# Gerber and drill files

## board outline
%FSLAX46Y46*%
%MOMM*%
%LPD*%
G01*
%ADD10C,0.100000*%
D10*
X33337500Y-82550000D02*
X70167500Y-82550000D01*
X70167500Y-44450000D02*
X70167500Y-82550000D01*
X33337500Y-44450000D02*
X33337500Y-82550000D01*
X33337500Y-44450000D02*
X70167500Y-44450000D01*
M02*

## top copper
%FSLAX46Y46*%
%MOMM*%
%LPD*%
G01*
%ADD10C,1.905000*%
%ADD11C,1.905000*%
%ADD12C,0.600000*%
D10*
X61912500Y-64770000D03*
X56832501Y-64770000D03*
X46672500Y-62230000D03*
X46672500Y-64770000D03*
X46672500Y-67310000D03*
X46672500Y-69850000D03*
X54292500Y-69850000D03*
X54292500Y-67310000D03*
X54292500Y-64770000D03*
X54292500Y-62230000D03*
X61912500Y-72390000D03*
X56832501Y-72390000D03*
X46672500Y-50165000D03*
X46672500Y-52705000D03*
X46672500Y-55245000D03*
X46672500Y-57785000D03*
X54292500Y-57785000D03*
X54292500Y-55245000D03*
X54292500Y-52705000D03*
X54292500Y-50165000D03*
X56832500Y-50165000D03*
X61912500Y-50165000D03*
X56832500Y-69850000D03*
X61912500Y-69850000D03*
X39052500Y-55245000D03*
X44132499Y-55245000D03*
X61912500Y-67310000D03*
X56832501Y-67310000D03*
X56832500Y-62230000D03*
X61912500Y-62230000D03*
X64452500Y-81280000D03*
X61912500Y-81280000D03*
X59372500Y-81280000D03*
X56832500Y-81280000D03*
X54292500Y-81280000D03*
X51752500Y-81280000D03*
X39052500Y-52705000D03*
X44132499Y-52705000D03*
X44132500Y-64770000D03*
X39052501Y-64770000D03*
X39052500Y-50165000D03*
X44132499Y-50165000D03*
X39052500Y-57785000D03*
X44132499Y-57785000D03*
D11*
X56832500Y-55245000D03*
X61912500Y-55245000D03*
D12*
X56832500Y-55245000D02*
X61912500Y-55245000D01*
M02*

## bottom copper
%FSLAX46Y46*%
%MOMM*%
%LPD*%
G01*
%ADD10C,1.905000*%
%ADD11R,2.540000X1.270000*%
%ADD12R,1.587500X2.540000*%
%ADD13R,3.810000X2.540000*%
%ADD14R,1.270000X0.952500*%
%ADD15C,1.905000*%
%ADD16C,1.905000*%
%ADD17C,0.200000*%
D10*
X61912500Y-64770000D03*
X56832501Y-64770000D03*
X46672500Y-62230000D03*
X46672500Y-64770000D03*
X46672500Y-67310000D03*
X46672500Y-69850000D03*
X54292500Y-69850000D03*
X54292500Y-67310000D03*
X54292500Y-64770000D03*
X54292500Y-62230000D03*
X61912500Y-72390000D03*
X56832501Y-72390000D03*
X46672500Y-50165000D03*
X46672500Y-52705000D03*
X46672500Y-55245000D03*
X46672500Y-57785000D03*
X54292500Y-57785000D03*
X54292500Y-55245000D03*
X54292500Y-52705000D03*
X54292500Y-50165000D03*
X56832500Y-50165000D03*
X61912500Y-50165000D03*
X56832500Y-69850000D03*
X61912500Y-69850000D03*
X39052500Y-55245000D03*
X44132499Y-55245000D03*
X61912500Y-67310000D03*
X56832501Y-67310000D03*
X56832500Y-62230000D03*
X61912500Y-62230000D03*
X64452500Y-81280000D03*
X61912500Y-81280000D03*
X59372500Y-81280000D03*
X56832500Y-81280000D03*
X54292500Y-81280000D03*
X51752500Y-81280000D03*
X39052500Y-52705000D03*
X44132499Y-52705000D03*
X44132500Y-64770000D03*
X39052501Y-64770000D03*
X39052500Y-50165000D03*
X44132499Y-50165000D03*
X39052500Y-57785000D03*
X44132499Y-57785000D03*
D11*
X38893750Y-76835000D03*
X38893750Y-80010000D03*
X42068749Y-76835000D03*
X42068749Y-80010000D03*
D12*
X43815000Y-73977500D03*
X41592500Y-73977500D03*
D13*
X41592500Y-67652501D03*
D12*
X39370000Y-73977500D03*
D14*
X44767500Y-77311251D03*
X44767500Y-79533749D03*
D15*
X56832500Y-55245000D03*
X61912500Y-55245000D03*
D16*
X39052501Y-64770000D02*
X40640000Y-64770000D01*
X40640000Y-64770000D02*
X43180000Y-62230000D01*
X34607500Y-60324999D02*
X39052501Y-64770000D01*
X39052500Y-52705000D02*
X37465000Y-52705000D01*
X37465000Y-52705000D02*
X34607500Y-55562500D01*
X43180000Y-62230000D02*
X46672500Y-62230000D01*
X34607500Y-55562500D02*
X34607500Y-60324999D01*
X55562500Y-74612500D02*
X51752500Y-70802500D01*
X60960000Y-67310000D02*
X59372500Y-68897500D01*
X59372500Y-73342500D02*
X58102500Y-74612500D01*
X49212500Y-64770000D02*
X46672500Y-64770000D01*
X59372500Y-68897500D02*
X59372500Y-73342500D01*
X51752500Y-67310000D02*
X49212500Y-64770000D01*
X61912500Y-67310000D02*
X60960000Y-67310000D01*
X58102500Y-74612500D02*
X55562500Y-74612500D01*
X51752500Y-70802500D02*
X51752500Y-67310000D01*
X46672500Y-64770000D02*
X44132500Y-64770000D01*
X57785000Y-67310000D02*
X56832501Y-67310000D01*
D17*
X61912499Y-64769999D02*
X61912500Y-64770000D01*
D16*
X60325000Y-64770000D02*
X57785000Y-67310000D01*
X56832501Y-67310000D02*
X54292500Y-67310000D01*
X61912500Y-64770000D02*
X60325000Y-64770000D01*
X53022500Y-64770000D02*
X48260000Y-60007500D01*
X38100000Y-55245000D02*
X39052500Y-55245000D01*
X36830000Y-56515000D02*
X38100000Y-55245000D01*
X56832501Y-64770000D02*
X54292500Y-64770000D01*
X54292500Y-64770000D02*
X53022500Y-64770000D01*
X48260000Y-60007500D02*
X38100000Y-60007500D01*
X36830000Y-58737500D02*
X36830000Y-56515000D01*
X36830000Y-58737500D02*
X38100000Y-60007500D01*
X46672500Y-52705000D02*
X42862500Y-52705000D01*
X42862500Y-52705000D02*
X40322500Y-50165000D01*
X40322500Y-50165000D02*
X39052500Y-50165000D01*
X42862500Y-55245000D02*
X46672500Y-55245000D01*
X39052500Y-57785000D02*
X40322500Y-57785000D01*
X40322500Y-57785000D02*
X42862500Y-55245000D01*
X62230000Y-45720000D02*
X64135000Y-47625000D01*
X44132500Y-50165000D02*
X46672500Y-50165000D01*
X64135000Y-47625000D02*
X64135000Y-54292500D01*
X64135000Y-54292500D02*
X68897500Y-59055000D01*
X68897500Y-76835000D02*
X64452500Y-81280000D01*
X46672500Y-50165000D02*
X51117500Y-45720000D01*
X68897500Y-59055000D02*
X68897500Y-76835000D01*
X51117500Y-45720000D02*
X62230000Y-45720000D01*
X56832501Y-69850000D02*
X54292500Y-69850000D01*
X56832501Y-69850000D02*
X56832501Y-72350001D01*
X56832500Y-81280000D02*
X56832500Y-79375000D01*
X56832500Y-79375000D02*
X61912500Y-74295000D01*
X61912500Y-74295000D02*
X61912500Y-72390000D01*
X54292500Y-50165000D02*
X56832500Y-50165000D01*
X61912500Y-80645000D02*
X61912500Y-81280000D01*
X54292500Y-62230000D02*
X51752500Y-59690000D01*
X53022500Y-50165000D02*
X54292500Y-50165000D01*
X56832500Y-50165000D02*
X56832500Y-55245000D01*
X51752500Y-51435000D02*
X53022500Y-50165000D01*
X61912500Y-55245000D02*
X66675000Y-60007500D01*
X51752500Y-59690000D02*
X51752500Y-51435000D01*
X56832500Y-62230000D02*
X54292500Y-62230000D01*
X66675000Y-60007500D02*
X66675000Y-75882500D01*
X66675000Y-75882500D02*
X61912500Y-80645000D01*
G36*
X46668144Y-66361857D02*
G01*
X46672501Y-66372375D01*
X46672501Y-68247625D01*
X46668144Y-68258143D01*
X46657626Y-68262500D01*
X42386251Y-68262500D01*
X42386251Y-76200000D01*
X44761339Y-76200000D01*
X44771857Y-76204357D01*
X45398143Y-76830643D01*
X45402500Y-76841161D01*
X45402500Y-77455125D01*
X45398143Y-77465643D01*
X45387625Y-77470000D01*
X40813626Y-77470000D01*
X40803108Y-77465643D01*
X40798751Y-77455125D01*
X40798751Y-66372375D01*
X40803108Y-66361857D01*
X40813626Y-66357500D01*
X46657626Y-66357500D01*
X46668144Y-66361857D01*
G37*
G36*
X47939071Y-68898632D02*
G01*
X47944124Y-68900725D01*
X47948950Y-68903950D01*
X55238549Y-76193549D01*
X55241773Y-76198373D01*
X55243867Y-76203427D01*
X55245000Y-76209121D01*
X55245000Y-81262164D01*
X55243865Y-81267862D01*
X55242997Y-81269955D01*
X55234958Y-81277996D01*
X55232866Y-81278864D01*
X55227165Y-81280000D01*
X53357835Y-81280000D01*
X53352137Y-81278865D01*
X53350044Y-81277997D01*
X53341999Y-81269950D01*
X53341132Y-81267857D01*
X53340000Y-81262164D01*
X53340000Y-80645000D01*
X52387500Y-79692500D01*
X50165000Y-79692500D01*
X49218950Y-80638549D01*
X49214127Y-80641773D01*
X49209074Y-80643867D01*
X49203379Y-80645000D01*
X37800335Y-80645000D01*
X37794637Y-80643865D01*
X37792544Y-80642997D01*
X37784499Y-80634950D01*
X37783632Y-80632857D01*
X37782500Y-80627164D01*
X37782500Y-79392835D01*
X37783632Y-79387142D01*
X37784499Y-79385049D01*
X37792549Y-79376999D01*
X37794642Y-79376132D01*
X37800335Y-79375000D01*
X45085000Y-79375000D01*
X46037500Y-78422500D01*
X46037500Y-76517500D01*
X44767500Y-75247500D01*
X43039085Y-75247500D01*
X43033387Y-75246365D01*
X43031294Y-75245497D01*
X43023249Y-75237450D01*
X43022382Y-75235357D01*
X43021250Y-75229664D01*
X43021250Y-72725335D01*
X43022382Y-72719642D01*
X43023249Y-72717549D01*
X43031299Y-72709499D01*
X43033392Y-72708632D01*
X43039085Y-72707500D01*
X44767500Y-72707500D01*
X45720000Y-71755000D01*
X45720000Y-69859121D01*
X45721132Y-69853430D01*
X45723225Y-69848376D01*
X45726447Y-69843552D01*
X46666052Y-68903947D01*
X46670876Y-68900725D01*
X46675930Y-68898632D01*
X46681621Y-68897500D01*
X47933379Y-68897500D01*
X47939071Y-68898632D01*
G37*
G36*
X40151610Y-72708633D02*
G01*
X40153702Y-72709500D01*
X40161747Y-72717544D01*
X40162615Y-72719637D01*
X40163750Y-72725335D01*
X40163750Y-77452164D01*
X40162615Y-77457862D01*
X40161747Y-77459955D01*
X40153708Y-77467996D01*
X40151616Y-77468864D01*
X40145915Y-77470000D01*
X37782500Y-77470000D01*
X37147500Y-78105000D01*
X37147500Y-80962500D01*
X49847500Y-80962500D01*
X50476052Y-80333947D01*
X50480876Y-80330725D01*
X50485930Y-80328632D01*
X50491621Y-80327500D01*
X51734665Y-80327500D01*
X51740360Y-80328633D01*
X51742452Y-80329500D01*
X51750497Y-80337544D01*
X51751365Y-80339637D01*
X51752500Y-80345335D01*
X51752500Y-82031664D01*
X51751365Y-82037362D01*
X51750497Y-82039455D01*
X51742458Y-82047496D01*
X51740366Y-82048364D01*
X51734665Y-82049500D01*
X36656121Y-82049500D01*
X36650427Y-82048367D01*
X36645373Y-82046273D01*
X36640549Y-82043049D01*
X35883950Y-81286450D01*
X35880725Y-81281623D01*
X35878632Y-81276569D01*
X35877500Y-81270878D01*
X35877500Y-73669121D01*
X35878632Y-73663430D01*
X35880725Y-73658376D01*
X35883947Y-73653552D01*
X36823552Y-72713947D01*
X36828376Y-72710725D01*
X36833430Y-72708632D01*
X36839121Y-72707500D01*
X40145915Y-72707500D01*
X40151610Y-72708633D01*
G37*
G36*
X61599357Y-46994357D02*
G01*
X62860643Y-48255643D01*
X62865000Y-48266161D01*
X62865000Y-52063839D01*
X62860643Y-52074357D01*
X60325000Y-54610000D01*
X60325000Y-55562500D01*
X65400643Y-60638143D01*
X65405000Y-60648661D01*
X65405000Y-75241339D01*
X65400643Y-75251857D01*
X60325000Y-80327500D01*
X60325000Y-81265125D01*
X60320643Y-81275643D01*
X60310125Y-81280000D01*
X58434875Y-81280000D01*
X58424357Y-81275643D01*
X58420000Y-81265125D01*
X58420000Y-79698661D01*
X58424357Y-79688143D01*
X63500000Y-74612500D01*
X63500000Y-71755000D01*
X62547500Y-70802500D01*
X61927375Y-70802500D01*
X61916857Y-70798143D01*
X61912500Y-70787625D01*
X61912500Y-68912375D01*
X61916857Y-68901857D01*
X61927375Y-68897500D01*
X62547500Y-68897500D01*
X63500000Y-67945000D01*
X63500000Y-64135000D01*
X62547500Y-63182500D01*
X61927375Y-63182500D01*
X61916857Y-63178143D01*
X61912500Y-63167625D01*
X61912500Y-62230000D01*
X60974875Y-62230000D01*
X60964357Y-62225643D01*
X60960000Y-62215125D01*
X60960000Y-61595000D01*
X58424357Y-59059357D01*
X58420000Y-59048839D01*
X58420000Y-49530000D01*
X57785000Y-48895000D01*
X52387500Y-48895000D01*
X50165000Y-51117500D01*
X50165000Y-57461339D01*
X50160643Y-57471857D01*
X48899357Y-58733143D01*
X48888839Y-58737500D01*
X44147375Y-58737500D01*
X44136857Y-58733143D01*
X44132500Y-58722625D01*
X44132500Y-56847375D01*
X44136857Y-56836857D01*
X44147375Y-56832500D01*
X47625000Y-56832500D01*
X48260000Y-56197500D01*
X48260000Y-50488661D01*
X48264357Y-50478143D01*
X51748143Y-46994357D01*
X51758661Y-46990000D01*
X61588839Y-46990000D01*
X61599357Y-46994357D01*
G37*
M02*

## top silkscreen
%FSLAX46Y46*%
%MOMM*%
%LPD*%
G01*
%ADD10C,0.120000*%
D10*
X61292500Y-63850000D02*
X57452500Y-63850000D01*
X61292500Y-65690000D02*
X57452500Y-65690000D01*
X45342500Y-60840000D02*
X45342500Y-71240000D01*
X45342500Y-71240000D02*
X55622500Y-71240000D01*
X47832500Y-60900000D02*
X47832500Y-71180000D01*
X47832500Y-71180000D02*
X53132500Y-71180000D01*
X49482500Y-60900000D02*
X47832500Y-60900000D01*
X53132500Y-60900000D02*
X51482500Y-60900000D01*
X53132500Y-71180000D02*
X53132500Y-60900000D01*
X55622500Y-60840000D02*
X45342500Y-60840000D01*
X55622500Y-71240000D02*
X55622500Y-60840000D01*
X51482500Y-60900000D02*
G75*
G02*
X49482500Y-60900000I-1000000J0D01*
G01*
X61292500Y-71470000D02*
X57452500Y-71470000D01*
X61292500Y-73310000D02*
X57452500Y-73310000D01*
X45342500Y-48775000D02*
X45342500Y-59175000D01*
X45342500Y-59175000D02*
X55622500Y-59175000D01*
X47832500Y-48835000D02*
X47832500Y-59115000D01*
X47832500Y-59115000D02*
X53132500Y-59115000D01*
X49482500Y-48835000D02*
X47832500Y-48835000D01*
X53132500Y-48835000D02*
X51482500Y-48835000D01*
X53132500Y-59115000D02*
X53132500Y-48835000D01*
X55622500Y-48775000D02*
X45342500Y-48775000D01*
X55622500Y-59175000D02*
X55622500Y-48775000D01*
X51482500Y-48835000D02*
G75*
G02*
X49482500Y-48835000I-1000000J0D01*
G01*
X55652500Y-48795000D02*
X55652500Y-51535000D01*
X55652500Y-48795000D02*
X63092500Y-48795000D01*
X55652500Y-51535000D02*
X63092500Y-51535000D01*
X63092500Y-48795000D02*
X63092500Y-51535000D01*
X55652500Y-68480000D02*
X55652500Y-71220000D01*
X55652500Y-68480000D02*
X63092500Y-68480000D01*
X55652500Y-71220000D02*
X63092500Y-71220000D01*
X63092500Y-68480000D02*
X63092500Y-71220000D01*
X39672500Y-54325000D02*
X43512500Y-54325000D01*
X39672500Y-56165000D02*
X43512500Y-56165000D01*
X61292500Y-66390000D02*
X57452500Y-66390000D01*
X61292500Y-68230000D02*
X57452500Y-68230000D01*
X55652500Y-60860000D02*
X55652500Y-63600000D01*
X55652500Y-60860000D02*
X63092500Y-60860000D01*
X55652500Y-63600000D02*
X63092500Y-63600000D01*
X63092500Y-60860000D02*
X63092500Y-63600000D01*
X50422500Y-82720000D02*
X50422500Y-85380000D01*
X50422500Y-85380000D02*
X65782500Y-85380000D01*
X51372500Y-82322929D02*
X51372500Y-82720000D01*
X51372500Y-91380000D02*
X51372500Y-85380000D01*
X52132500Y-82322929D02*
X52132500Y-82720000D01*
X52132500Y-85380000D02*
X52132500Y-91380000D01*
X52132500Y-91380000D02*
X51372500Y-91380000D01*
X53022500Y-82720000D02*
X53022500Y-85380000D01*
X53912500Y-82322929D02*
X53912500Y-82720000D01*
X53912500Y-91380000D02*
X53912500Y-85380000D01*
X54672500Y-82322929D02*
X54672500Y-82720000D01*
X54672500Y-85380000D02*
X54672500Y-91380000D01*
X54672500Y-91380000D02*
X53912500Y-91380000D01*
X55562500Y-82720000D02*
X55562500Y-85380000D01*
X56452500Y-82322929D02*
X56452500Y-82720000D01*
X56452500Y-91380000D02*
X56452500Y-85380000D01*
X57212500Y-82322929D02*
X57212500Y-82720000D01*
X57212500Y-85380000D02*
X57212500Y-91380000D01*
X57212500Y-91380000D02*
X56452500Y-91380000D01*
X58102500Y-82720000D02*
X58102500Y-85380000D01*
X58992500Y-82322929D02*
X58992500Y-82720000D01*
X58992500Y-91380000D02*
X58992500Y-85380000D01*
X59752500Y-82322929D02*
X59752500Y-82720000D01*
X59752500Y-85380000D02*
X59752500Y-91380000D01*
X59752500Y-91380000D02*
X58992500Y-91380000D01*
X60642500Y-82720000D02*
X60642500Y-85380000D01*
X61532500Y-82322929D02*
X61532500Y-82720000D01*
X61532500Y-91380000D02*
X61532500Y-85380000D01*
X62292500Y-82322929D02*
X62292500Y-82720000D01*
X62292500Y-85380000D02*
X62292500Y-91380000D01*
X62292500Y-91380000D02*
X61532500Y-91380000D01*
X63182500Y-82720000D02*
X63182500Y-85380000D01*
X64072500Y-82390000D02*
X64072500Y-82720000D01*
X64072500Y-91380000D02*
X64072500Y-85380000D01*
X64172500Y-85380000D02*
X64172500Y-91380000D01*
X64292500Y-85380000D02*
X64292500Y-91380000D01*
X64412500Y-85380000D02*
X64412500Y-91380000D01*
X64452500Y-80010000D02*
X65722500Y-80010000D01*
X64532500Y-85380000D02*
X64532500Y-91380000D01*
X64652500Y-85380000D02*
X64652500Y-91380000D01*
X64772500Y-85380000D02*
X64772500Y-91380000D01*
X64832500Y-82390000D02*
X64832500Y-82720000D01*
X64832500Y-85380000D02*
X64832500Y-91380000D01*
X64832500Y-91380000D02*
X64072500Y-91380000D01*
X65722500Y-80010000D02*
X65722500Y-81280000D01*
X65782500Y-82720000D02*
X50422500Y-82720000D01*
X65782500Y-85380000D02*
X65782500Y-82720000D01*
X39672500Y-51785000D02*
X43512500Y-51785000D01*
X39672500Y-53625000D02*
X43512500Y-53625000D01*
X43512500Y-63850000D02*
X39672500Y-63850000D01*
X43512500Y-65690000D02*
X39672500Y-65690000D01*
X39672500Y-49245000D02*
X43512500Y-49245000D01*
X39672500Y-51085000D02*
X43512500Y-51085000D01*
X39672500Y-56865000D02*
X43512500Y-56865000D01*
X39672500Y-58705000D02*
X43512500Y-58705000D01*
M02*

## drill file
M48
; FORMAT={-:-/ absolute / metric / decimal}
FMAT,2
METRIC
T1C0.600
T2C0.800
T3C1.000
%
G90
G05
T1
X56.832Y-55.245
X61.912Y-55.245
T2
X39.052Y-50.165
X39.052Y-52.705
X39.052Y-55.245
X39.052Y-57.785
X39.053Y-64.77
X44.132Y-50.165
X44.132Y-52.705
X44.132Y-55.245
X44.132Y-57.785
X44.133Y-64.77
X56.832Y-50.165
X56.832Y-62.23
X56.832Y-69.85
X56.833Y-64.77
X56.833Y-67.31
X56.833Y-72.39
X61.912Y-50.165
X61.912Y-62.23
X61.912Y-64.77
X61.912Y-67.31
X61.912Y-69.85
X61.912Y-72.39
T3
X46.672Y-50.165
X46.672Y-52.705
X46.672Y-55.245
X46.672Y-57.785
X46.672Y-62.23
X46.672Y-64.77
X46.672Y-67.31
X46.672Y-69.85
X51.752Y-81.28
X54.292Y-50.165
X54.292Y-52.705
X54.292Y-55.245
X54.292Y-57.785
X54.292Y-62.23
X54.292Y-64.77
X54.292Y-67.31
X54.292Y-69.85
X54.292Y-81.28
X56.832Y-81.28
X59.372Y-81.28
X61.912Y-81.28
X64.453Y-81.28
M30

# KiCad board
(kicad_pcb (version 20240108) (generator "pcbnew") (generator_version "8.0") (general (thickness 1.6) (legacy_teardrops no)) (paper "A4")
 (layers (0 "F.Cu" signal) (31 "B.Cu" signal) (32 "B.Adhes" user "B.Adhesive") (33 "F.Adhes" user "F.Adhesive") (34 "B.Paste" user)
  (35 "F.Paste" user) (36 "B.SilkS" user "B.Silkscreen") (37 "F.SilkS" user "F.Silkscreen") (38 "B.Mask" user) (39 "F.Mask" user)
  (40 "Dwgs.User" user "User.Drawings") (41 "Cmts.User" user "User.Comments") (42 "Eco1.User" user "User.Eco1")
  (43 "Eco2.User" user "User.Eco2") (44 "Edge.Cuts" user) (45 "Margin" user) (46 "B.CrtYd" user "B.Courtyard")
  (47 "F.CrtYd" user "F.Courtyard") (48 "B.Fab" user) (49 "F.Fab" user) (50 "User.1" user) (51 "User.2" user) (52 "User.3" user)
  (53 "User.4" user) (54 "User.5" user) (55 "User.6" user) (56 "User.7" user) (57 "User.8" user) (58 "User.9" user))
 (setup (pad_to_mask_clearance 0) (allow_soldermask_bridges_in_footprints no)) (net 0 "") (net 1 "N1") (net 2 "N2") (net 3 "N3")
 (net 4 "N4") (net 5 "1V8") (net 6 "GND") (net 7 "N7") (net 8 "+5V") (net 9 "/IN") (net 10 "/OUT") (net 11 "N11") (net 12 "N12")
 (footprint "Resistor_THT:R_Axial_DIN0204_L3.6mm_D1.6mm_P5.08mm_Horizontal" (layer "F.Cu") (at 61.9125 64.77 180)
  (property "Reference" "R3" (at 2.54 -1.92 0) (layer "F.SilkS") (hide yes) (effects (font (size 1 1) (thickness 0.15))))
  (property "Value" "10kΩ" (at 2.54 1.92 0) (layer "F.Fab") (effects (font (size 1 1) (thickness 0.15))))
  (fp_line (start 0.62 0.92) (end 4.46 0.92) (stroke (width 0.12) (type solid)) (layer "F.SilkS"))
  (fp_line (start 0.62 -0.92) (end 4.46 -0.92) (stroke (width 0.12) (type solid)) (layer "F.SilkS"))
  (pad "1" thru_hole circle (at 0 0 180) (size 1.905 1.905) (drill 0.8) (layers "*.Cu" "*.Mask") (remove_unused_layers no) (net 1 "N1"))
  (pad "2" thru_hole circle (at 5.079999 0 180) (size 1.905 1.905) (drill 0.8) (layers "*.Cu" "*.Mask") (remove_unused_layers no)
   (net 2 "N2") (thermal_bridge_angle 90)))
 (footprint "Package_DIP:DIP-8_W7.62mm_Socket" (layer "F.Cu") (at 50.4825 66.04)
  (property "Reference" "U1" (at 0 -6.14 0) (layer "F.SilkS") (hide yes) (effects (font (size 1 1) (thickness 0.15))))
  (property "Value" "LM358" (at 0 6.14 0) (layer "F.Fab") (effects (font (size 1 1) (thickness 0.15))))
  (fp_line (start -5.14 -5.2) (end -5.14 5.2) (stroke (width 0.12) (type solid)) (layer "F.SilkS"))
  (fp_line (start -5.14 5.2) (end 5.14 5.2) (stroke (width 0.12) (type solid)) (layer "F.SilkS"))
  (fp_line (start -2.65 -5.14) (end -2.65 5.14) (stroke (width 0.12) (type solid)) (layer "F.SilkS"))
  (fp_line (start -2.65 5.14) (end 2.65 5.14) (stroke (width 0.12) (type solid)) (layer "F.SilkS"))
  (fp_line (start -1 -5.14) (end -2.65 -5.14) (stroke (width 0.12) (type solid)) (layer "F.SilkS"))
  (fp_line (start 2.65 -5.14) (end 1 -5.14) (stroke (width 0.12) (type solid)) (layer "F.SilkS"))
  (fp_line (start 2.65 5.14) (end 2.65 -5.14) (stroke (width 0.12) (type solid)) (layer "F.SilkS"))
  (fp_line (start 5.14 -5.2) (end -5.14 -5.2) (stroke (width 0.12) (type solid)) (layer "F.SilkS"))
  (fp_line (start 5.14 5.2) (end 5.14 -5.2) (stroke (width 0.12) (type solid)) (layer "F.SilkS"))
  (fp_arc (start 1 -5.14) (mid 0 -4.14) (end -1 -5.14) (stroke (width 0.12) (type solid)) (layer "F.SilkS"))
  (pad "1" thru_hole circle (at -3.81 -3.81) (size 1.905 1.905) (drill 1) (layers "*.Cu" "*.Mask") (remove_unused_layers no) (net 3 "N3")
   (thermal_bridge_angle 90))
  (pad "2" thru_hole circle (at -3.81 -1.27) (size 1.905 1.905) (drill 1) (layers "*.Cu" "*.Mask") (remove_unused_layers no) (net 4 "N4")
   (thermal_bridge_angle 90))
  (pad "3" thru_hole circle (at -3.81 1.27) (size 1.905 1.905) (drill 1) (layers "*.Cu" "*.Mask") (remove_unused_layers no) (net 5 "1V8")
   (thermal_bridge_angle 90))
  (pad "4" thru_hole circle (at -3.81 3.81) (size 1.905 1.905) (drill 1) (layers "*.Cu" "*.Mask") (remove_unused_layers no) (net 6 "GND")
   (thermal_bridge_angle 90))
  (pad "5" thru_hole circle (at 3.81 3.81) (size 1.905 1.905) (drill 1) (layers "*.Cu" "*.Mask") (remove_unused_layers no) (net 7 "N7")
   (thermal_bridge_angle 90))
  (pad "6" thru_hole circle (at 3.81 1.27) (size 1.905 1.905) (drill 1) (layers "*.Cu" "*.Mask") (remove_unused_layers no) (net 1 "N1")
   (thermal_bridge_angle 90))
  (pad "7" thru_hole circle (at 3.81 -1.27) (size 1.905 1.905) (drill 1) (layers "*.Cu" "*.Mask") (remove_unused_layers no) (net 2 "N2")
   (thermal_bridge_angle 90))
  (pad "8" thru_hole circle (at 3.81 -3.81) (size 1.905 1.905) (drill 1) (layers "*.Cu" "*.Mask") (remove_unused_layers no) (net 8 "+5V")
   (thermal_bridge_angle 90)))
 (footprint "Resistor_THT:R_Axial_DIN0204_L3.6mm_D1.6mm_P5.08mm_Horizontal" (layer "F.Cu") (at 61.9125 72.39 180)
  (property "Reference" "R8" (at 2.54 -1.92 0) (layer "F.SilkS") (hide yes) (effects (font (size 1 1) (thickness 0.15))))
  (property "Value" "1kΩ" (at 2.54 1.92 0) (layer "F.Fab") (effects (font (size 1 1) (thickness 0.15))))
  (fp_line (start 0.62 0.92) (end 4.46 0.92) (stroke (width 0.12) (type solid)) (layer "F.SilkS"))
  (fp_line (start 0.62 -0.92) (end 4.46 -0.92) (stroke (width 0.12) (type solid)) (layer "F.SilkS"))
  (pad "1" thru_hole circle (at 0 0 180) (size 1.905 1.905) (drill 0.8) (layers "*.Cu" "*.Mask") (remove_unused_layers no) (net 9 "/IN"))
  (pad "2" thru_hole circle (at 5.079999 0 180) (size 1.905 1.905) (drill 0.8) (layers "*.Cu" "*.Mask") (remove_unused_layers no)
   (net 7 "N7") (thermal_bridge_angle 90)))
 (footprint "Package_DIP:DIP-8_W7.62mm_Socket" (layer "F.Cu") (at 50.4825 53.975)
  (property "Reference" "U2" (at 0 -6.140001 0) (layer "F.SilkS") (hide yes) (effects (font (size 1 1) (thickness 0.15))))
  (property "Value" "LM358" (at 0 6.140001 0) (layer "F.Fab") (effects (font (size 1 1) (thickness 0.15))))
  (fp_line (start -5.14 -5.2) (end -5.14 5.2) (stroke (width 0.12) (type solid)) (layer "F.SilkS"))
  (fp_line (start -5.14 5.2) (end 5.14 5.2) (stroke (width 0.12) (type solid)) (layer "F.SilkS"))
  (fp_line (start -2.65 -5.14) (end -2.65 5.14) (stroke (width 0.12) (type solid)) (layer "F.SilkS"))
  (fp_line (start -2.65 5.14) (end 2.65 5.14) (stroke (width 0.12) (type solid)) (layer "F.SilkS"))
  (fp_line (start -1 -5.14) (end -2.65 -5.14) (stroke (width 0.12) (type solid)) (layer "F.SilkS"))
  (fp_line (start 2.65 -5.14) (end 1 -5.14) (stroke (width 0.12) (type solid)) (layer "F.SilkS"))
  (fp_line (start 2.65 5.14) (end 2.65 -5.14) (stroke (width 0.12) (type solid)) (layer "F.SilkS"))
  (fp_line (start 5.14 -5.2) (end -5.14 -5.2) (stroke (width 0.12) (type solid)) (layer "F.SilkS"))
  (fp_line (start 5.14 5.2) (end 5.14 -5.2) (stroke (width 0.12) (type solid)) (layer "F.SilkS"))
  (fp_arc (start 1 -5.14) (mid 0 -4.14) (end -1 -5.14) (stroke (width 0.12) (type solid)) (layer "F.SilkS"))
  (pad "1" thru_hole circle (at -3.81 -3.81) (size 1.905 1.905) (drill 1) (layers "*.Cu" "*.Mask") (remove_unused_layers no) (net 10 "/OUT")
   (thermal_bridge_angle 90))
  (pad "2" thru_hole circle (at -3.81 -1.27) (size 1.905 1.905) (drill 1) (layers "*.Cu" "*.Mask") (remove_unused_layers no) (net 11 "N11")
   (thermal_bridge_angle 90))
  (pad "3" thru_hole circle (at -3.81 1.27) (size 1.905 1.905) (drill 1) (layers "*.Cu" "*.Mask") (remove_unused_layers no) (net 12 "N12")
   (thermal_bridge_angle 90))
  (pad "4" thru_hole circle (at -3.81 3.81) (size 1.905 1.905) (drill 1) (layers "*.Cu" "*.Mask") (remove_unused_layers no) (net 6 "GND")
   (thermal_bridge_angle 90))
  (pad "5" thru_hole circle (at 3.81 3.81) (size 1.905 1.905) (drill 1) (layers "*.Cu" "*.Mask") (remove_unused_layers no)
   (thermal_bridge_angle 90))
  (pad "6" thru_hole circle (at 3.81 1.27) (size 1.905 1.905) (drill 1) (layers "*.Cu" "*.Mask") (remove_unused_layers no)
   (thermal_bridge_angle 90))
  (pad "7" thru_hole circle (at 3.81 -1.27) (size 1.905 1.905) (drill 1) (layers "*.Cu" "*.Mask") (remove_unused_layers no)
   (thermal_bridge_angle 90))
  (pad "8" thru_hole circle (at 3.81 -3.81) (size 1.905 1.905) (drill 1) (layers "*.Cu" "*.Mask") (remove_unused_layers no) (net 8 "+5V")
   (thermal_bridge_angle 90)))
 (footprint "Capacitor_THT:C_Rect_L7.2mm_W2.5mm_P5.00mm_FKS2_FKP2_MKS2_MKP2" (layer "F.Cu") (at 56.8725 50.165)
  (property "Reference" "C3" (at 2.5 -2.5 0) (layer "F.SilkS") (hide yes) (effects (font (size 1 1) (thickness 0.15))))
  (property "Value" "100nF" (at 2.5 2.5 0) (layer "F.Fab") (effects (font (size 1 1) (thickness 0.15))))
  (fp_line (start -1.22 -1.37) (end -1.22 1.37) (stroke (width 0.12) (type solid)) (layer "F.SilkS"))
  (fp_line (start -1.22 -1.37) (end 6.22 -1.37) (stroke (width 0.12) (type solid)) (layer "F.SilkS"))
  (fp_line (start -1.22 1.37) (end 6.22 1.37) (stroke (width 0.12) (type solid)) (layer "F.SilkS"))
  (fp_line (start 6.22 -1.37) (end 6.22 1.37) (stroke (width 0.12) (type solid)) (layer "F.SilkS"))
  (pad "1" thru_hole circle (at -0.04 0) (size 1.905 1.6) (drill 0.8) (layers "*.Cu" "*.Mask") (remove_unused_layers no) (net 8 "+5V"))
  (pad "2" thru_hole circle (at 5.04 0) (size 1.905 1.6) (drill 0.8) (layers "*.Cu" "*.Mask") (remove_unused_layers no) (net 6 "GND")))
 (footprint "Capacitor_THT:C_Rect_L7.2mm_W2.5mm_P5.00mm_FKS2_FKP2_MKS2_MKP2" (layer "F.Cu") (at 56.8725 69.85)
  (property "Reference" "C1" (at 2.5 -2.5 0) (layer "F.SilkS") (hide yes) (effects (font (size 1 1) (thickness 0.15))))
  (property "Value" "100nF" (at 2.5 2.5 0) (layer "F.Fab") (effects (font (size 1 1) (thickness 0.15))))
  (fp_line (start -1.22 -1.37) (end -1.22 1.37) (stroke (width 0.12) (type solid)) (layer "F.SilkS"))
  (fp_line (start -1.22 -1.37) (end 6.22 -1.37) (stroke (width 0.12) (type solid)) (layer "F.SilkS"))
  (fp_line (start -1.22 1.37) (end 6.22 1.37) (stroke (width 0.12) (type solid)) (layer "F.SilkS"))
  (fp_line (start 6.22 -1.37) (end 6.22 1.37) (stroke (width 0.12) (type solid)) (layer "F.SilkS"))
  (pad "1" thru_hole circle (at -0.04 0) (size 1.905 1.6) (drill 0.8) (layers "*.Cu" "*.Mask") (remove_unused_layers no) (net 7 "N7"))
  (pad "2" thru_hole circle (at 5.04 0) (size 1.905 1.6) (drill 0.8) (layers "*.Cu" "*.Mask") (remove_unused_layers no) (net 6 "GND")))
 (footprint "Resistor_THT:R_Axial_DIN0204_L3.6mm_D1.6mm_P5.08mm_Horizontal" (layer "F.Cu") (at 39.0525 55.245)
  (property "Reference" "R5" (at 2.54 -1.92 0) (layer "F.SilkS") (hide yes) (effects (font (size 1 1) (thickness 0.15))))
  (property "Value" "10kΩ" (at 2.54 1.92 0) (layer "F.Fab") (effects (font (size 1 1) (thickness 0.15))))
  (fp_line (start 0.62 -0.92) (end 4.46 -0.92) (stroke (width 0.12) (type solid)) (layer "F.SilkS"))
  (fp_line (start 0.62 0.92) (end 4.46 0.92) (stroke (width 0.12) (type solid)) (layer "F.SilkS"))
  (pad "1" thru_hole circle (at 0 0) (size 1.905 1.905) (drill 0.8) (layers "*.Cu" "*.Mask") (remove_unused_layers no) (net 2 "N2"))
  (pad "2" thru_hole circle (at 5.079999 0) (size 1.905 1.905) (drill 0.8) (layers "*.Cu" "*.Mask") (remove_unused_layers no) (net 12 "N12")
   (thermal_bridge_angle 90)))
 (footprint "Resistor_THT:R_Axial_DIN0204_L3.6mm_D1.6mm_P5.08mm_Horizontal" (layer "F.Cu") (at 61.9125 67.31 180)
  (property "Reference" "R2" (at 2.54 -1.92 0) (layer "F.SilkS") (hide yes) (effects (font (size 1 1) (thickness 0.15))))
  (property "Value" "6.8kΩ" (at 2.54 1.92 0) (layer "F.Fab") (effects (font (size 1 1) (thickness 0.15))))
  (fp_line (start 0.62 0.92) (end 4.46 0.92) (stroke (width 0.12) (type solid)) (layer "F.SilkS"))
  (fp_line (start 0.62 -0.92) (end 4.46 -0.92) (stroke (width 0.12) (type solid)) (layer "F.SilkS"))
  (pad "1" thru_hole circle (at 0 0 180) (size 1.905 1.905) (drill 0.8) (layers "*.Cu" "*.Mask") (remove_unused_layers no) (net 4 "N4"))
  (pad "2" thru_hole circle (at 5.079999 0 180) (size 1.905 1.905) (drill 0.8) (layers "*.Cu" "*.Mask") (remove_unused_layers no)
   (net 1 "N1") (thermal_bridge_angle 90)))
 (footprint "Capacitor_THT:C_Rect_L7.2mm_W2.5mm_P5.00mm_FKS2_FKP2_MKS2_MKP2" (layer "F.Cu") (at 56.8725 62.23)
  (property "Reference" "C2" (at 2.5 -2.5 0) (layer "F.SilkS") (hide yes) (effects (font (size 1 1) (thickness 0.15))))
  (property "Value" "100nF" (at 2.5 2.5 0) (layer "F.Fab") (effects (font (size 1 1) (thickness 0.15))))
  (fp_line (start -1.22 -1.37) (end -1.22 1.37) (stroke (width 0.12) (type solid)) (layer "F.SilkS"))
  (fp_line (start -1.22 -1.37) (end 6.22 -1.37) (stroke (width 0.12) (type solid)) (layer "F.SilkS"))
  (fp_line (start -1.22 1.37) (end 6.22 1.37) (stroke (width 0.12) (type solid)) (layer "F.SilkS"))
  (fp_line (start 6.22 -1.37) (end 6.22 1.37) (stroke (width 0.12) (type solid)) (layer "F.SilkS"))
  (pad "1" thru_hole circle (at -0.04 0) (size 1.905 1.6) (drill 0.8) (layers "*.Cu" "*.Mask") (remove_unused_layers no) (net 8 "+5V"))
  (pad "2" thru_hole circle (at 5.04 0) (size 1.905 1.6) (drill 0.8) (layers "*.Cu" "*.Mask") (remove_unused_layers no) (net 6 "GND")))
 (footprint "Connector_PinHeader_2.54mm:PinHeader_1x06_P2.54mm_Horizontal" (layer "F.Cu") (at 64.4525 81.28 -90)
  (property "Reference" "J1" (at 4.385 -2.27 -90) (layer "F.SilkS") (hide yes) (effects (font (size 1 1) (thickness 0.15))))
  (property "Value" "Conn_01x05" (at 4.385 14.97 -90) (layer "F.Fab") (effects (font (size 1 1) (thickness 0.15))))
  (fp_line (start 1.44 14.03) (end 4.1 14.03) (stroke (width 0.12) (type solid)) (layer "F.SilkS"))
  (fp_line (start 4.1 14.03) (end 4.1 -1.33) (stroke (width 0.12) (type solid)) (layer "F.SilkS"))
  (fp_line (start 1.042929 13.08) (end 1.44 13.08) (stroke (width 0.12) (type solid)) (layer "F.SilkS"))
  (fp_line (start 10.1 13.08) (end 4.1 13.08) (stroke (width 0.12) (type solid)) (layer "F.SilkS"))
  (fp_line (start 1.042929 12.32) (end 1.44 12.32) (stroke (width 0.12) (type solid)) (layer "F.SilkS"))
  (fp_line (start 4.1 12.32) (end 10.1 12.32) (stroke (width 0.12) (type solid)) (layer "F.SilkS"))
  (fp_line (start 10.1 12.32) (end 10.1 13.08) (stroke (width 0.12) (type solid)) (layer "F.SilkS"))
  (fp_line (start 1.44 11.43) (end 4.1 11.43) (stroke (width 0.12) (type solid)) (layer "F.SilkS"))
  (fp_line (start 1.042929 10.54) (end 1.44 10.54) (stroke (width 0.12) (type solid)) (layer "F.SilkS"))
  (fp_line (start 10.1 10.54) (end 4.1 10.54) (stroke (width 0.12) (type solid)) (layer "F.SilkS"))
  (fp_line (start 1.042929 9.78) (end 1.44 9.78) (stroke (width 0.12) (type solid)) (layer "F.SilkS"))
  (fp_line (start 4.1 9.78) (end 10.1 9.78) (stroke (width 0.12) (type solid)) (layer "F.SilkS"))
  (fp_line (start 10.1 9.78) (end 10.1 10.54) (stroke (width 0.12) (type solid)) (layer "F.SilkS"))
  (fp_line (start 1.44 8.89) (end 4.1 8.89) (stroke (width 0.12) (type solid)) (layer "F.SilkS"))
  (fp_line (start 1.042929 8) (end 1.44 8) (stroke (width 0.12) (type solid)) (layer "F.SilkS"))
  (fp_line (start 10.1 8) (end 4.1 8) (stroke (width 0.12) (type solid)) (layer "F.SilkS"))
  (fp_line (start 1.042929 7.24) (end 1.44 7.24) (stroke (width 0.12) (type solid)) (layer "F.SilkS"))
  (fp_line (start 4.1 7.24) (end 10.1 7.24) (stroke (width 0.12) (type solid)) (layer "F.SilkS"))
  (fp_line (start 10.1 7.24) (end 10.1 8) (stroke (width 0.12) (type solid)) (layer "F.SilkS"))
  (fp_line (start 1.44 6.35) (end 4.1 6.35) (stroke (width 0.12) (type solid)) (layer "F.SilkS"))
  (fp_line (start 1.042929 5.46) (end 1.44 5.46) (stroke (width 0.12) (type solid)) (layer "F.SilkS"))
  (fp_line (start 10.1 5.46) (end 4.1 5.46) (stroke (width 0.12) (type solid)) (layer "F.SilkS"))
  (fp_line (start 1.042929 4.7) (end 1.44 4.7) (stroke (width 0.12) (type solid)) (layer "F.SilkS"))
  (fp_line (start 4.1 4.7) (end 10.1 4.7) (stroke (width 0.12) (type solid)) (layer "F.SilkS"))
  (fp_line (start 10.1 4.7) (end 10.1 5.46) (stroke (width 0.12) (type solid)) (layer "F.SilkS"))
  (fp_line (start 1.44 3.81) (end 4.1 3.81) (stroke (width 0.12) (type solid)) (layer "F.SilkS"))
  (fp_line (start 1.042929 2.92) (end 1.44 2.92) (stroke (width 0.12) (type solid)) (layer "F.SilkS"))
  (fp_line (start 10.1 2.92) (end 4.1 2.92) (stroke (width 0.12) (type solid)) (layer "F.SilkS"))
  (fp_line (start 1.042929 2.16) (end 1.44 2.16) (stroke (width 0.12) (type solid)) (layer "F.SilkS"))
  (fp_line (start 4.1 2.16) (end 10.1 2.16) (stroke (width 0.12) (type solid)) (layer "F.SilkS"))
  (fp_line (start 10.1 2.16) (end 10.1 2.92) (stroke (width 0.12) (type solid)) (layer "F.SilkS"))
  (fp_line (start 1.44 1.27) (end 4.1 1.27) (stroke (width 0.12) (type solid)) (layer "F.SilkS"))
  (fp_line (start 1.11 0.38) (end 1.44 0.38) (stroke (width 0.12) (type solid)) (layer "F.SilkS"))
  (fp_line (start 10.1 0.38) (end 4.1 0.38) (stroke (width 0.12) (type solid)) (layer "F.SilkS"))
  (fp_line (start 4.1 0.28) (end 10.1 0.28) (stroke (width 0.12) (type solid)) (layer "F.SilkS"))
  (fp_line (start 4.1 0.16) (end 10.1 0.16) (stroke (width 0.12) (type solid)) (layer "F.SilkS"))
  (fp_line (start 4.1 0.04) (end 10.1 0.04) (stroke (width 0.12) (type solid)) (layer "F.SilkS"))
  (fp_line (start -1.27 0) (end -1.27 -1.27) (stroke (width 0.12) (type solid)) (layer "F.SilkS"))
  (fp_line (start 4.1 -0.08) (end 10.1 -0.08) (stroke (width 0.12) (type solid)) (layer "F.SilkS"))
  (fp_line (start 4.1 -0.2) (end 10.1 -0.2) (stroke (width 0.12) (type solid)) (layer "F.SilkS"))
  (fp_line (start 4.1 -0.32) (end 10.1 -0.32) (stroke (width 0.12) (type solid)) (layer "F.SilkS"))
  (fp_line (start 1.11 -0.38) (end 1.44 -0.38) (stroke (width 0.12) (type solid)) (layer "F.SilkS"))
  (fp_line (start 4.1 -0.38) (end 10.1 -0.38) (stroke (width 0.12) (type solid)) (layer "F.SilkS"))
  (fp_line (start 10.1 -0.38) (end 10.1 0.38) (stroke (width 0.12) (type solid)) (layer "F.SilkS"))
  (fp_line (start -1.27 -1.27) (end 0 -1.27) (stroke (width 0.12) (type solid)) (layer "F.SilkS"))
  (fp_line (start 1.44 -1.33) (end 1.44 14.03) (stroke (width 0.12) (type solid)) (layer "F.SilkS"))
  (fp_line (start 4.1 -1.33) (end 1.44 -1.33) (stroke (width 0.12) (type solid)) (layer "F.SilkS"))
  (pad "1" thru_hole circle (at 0 0 270) (size 1.905 1.905) (drill 1) (layers "*.Cu" "*.Mask") (remove_unused_layers no) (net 10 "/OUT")
   (thermal_bridge_angle 90))
  (pad "2" thru_hole circle (at 0 2.54 270) (size 1.905 1.905) (drill 1) (layers "*.Cu" "*.Mask") (remove_unused_layers no) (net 8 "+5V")
   (thermal_bridge_angle 90))
  (pad "3" thru_hole circle (at 0 5.08 270) (size 1.905 1.905) (drill 1) (layers "*.Cu" "*.Mask") (remove_unused_layers no) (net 6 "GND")
   (thermal_bridge_angle 90))
  (pad "4" thru_hole circle (at 0 7.62 270) (size 1.905 1.905) (drill 1) (layers "*.Cu" "*.Mask") (remove_unused_layers no) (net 9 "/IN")
   (thermal_bridge_angle 90))
  (pad "5" thru_hole circle (at 0 10.16 270) (size 1.905 1.905) (drill 1) (layers "*.Cu" "*.Mask") (remove_unused_layers no) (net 6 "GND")
   (thermal_bridge_angle 90))
  (pad "6" thru_hole circle (at 0 12.7 270) (size 1.905 1.905) (drill 1) (layers "*.Cu" "*.Mask") (remove_unused_layers no) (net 8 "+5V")
   (thermal_bridge_angle 90)))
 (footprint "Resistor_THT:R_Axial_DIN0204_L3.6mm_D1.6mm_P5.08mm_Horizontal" (layer "F.Cu") (at 39.0525 52.705)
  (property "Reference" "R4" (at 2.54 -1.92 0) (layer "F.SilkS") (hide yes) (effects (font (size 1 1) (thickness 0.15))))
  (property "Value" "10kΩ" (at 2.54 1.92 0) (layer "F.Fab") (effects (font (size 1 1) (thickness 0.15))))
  (fp_line (start 0.62 -0.92) (end 4.46 -0.92) (stroke (width 0.12) (type solid)) (layer "F.SilkS"))
  (fp_line (start 0.62 0.92) (end 4.46 0.92) (stroke (width 0.12) (type solid)) (layer "F.SilkS"))
  (pad "1" thru_hole circle (at 0 0) (size 1.905 1.905) (drill 0.8) (layers "*.Cu" "*.Mask") (remove_unused_layers no) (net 3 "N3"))
  (pad "2" thru_hole circle (at 5.079999 0) (size 1.905 1.905) (drill 0.8) (layers "*.Cu" "*.Mask") (remove_unused_layers no) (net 11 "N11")
   (thermal_bridge_angle 90)))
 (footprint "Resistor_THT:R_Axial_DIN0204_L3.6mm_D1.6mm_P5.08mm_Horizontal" (layer "F.Cu") (at 44.1325 64.77 180)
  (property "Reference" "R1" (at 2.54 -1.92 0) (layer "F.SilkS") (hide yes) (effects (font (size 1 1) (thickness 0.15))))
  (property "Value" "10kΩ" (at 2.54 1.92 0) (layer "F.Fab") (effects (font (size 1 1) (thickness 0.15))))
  (fp_line (start 0.62 0.92) (end 4.46 0.92) (stroke (width 0.12) (type solid)) (layer "F.SilkS"))
  (fp_line (start 0.62 -0.92) (end 4.46 -0.92) (stroke (width 0.12) (type solid)) (layer "F.SilkS"))
  (pad "1" thru_hole circle (at 0 0 180) (size 1.905 1.905) (drill 0.8) (layers "*.Cu" "*.Mask") (remove_unused_layers no) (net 4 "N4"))
  (pad "2" thru_hole circle (at 5.079999 0 180) (size 1.905 1.905) (drill 0.8) (layers "*.Cu" "*.Mask") (remove_unused_layers no)
   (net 3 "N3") (thermal_bridge_angle 90)))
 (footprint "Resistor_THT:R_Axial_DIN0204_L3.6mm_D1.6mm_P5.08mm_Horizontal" (layer "F.Cu") (at 39.0525 50.165)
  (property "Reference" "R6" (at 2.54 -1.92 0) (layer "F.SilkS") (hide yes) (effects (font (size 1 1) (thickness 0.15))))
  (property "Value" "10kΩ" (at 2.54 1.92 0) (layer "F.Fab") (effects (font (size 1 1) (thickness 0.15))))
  (fp_line (start 0.62 -0.92) (end 4.46 -0.92) (stroke (width 0.12) (type solid)) (layer "F.SilkS"))
  (fp_line (start 0.62 0.92) (end 4.46 0.92) (stroke (width 0.12) (type solid)) (layer "F.SilkS"))
  (pad "1" thru_hole circle (at 0 0) (size 1.905 1.905) (drill 0.8) (layers "*.Cu" "*.Mask") (remove_unused_layers no) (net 11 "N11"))
  (pad "2" thru_hole circle (at 5.079999 0) (size 1.905 1.905) (drill 0.8) (layers "*.Cu" "*.Mask") (remove_unused_layers no)
   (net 10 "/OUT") (thermal_bridge_angle 90)))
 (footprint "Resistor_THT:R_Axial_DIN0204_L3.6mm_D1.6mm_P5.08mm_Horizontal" (layer "F.Cu") (at 39.0525 57.785)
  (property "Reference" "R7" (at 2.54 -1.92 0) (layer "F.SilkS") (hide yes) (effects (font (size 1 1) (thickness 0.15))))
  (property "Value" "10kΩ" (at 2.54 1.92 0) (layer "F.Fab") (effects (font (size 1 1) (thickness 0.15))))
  (fp_line (start 0.62 -0.92) (end 4.46 -0.92) (stroke (width 0.12) (type solid)) (layer "F.SilkS"))
  (fp_line (start 0.62 0.92) (end 4.46 0.92) (stroke (width 0.12) (type solid)) (layer "F.SilkS"))
  (pad "1" thru_hole circle (at 0 0) (size 1.905 1.905) (drill 0.8) (layers "*.Cu" "*.Mask") (remove_unused_layers no) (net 12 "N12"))
  (pad "2" thru_hole circle (at 5.079999 0) (size 1.905 1.905) (drill 0.8) (layers "*.Cu" "*.Mask") (remove_unused_layers no) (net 6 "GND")
   (thermal_bridge_angle 90)))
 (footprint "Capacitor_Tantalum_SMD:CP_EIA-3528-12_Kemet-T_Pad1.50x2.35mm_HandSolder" (layer "B.Cu") (at 38.89375 78.4225 -90)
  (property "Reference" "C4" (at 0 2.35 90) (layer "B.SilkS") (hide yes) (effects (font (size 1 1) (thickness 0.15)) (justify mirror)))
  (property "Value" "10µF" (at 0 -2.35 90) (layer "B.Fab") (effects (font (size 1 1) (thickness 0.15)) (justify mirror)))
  (pad "1" smd rect (at -1.5875 0 270) (size 1.27 2.54) (layers "B.Cu" "B.Paste" "B.Mask") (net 8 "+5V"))
  (pad "2" smd rect (at 1.5875 0 270) (size 1.27 2.54) (layers "B.Cu" "B.Paste" "B.Mask") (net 6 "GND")))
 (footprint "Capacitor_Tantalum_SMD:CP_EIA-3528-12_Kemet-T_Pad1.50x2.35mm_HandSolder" (layer "B.Cu") (at 42.068749 78.4225 -90)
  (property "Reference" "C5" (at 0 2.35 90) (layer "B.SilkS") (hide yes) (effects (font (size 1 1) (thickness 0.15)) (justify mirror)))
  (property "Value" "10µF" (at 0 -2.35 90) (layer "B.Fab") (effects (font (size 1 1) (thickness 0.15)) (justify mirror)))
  (pad "1" smd rect (at -1.5875 0 270) (size 1.27 2.54) (layers "B.Cu" "B.Paste" "B.Mask") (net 5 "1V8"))
  (pad "2" smd rect (at 1.5875 0 270) (size 1.27 2.54) (layers "B.Cu" "B.Paste" "B.Mask") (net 6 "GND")))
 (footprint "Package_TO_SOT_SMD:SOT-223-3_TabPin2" (layer "B.Cu") (at 41.5925 70.8025 90)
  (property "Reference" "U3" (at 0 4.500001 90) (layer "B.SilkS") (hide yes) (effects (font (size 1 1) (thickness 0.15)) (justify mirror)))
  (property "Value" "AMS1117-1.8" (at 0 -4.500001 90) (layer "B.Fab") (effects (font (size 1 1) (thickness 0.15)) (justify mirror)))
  (pad "1" smd rect (at -3.175 2.2225 90) (size 2.54 1.5875) (layers "B.Cu" "B.Paste" "B.Mask") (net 6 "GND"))
  (pad "2" smd rect (at -3.175 0 90) (size 2.54 1.5875) (layers "B.Cu" "B.Paste" "B.Mask") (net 5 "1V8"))
  (pad "2" smd rect (at 3.149999 0 90) (size 2.54 3.81) (layers "B.Cu" "B.Paste" "B.Mask") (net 5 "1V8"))
  (pad "3" smd rect (at -3.175 -2.2225 90) (size 2.54 1.5875) (layers "B.Cu" "B.Paste" "B.Mask") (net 8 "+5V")))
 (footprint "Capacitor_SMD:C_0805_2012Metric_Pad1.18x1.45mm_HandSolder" (layer "B.Cu") (at 44.7675 78.4225 -90)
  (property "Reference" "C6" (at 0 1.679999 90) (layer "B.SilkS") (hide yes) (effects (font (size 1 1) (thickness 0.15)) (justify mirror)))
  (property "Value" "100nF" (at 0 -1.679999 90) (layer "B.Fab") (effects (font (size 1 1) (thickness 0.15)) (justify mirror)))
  (pad "1" smd rect (at -1.111249 0 270) (size 0.9525 1.27) (layers "B.Cu" "B.Paste" "B.Mask") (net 5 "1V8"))
  (pad "2" smd rect (at 1.111249 0 270) (size 0.9525 1.27) (layers "B.Cu" "B.Paste" "B.Mask") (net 6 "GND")))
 (gr_line (start 33.3375 82.55) (end 70.1675 82.55) (stroke (width 0) (type default)) (layer "Edge.Cuts"))
 (gr_line (start 70.1675 44.45) (end 70.1675 82.55) (stroke (width 0) (type default)) (layer "Edge.Cuts"))
 (gr_line (start 33.3375 44.45) (end 33.3375 82.55) (stroke (width 0) (type default)) (layer "Edge.Cuts"))
 (gr_line (start 33.3375 44.45) (end 70.1675 44.45) (stroke (width 0) (type default)) (layer "Edge.Cuts"))
 (segment (start 39.052501 64.77) (end 40.64 64.77) (width 1.905) (layer "B.Cu") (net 3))
 (segment (start 40.64 64.77) (end 43.18 62.23) (width 1.905) (layer "B.Cu") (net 3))
 (segment (start 34.6075 60.324999) (end 39.052501 64.77) (width 1.905) (layer "B.Cu") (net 3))
 (segment (start 39.0525 52.705) (end 37.465 52.705) (width 1.905) (layer "B.Cu") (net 3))
 (segment (start 37.465 52.705) (end 34.6075 55.5625) (width 1.905) (layer "B.Cu") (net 3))
 (segment (start 43.18 62.23) (end 46.6725 62.23) (width 1.905) (layer "B.Cu") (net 3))
 (segment (start 34.6075 55.5625) (end 34.6075 60.324999) (width 1.905) (layer "B.Cu") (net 3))
 (segment (start 55.5625 74.6125) (end 51.7525 70.8025) (width 1.905) (layer "B.Cu") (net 4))
 (segment (start 60.96 67.31) (end 59.3725 68.8975) (width 1.905) (layer "B.Cu") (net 4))
 (segment (start 59.3725 73.3425) (end 58.1025 74.6125) (width 1.905) (layer "B.Cu") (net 4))
 (segment (start 49.2125 64.77) (end 46.6725 64.77) (width 1.905) (layer "B.Cu") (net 4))
 (segment (start 59.3725 68.8975) (end 59.3725 73.3425) (width 1.905) (layer "B.Cu") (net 4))
 (segment (start 51.7525 67.31) (end 49.2125 64.77) (width 1.905) (layer "B.Cu") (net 4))
 (segment (start 61.9125 67.31) (end 60.96 67.31) (width 1.905) (layer "B.Cu") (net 4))
 (segment (start 58.1025 74.6125) (end 55.5625 74.6125) (width 1.905) (layer "B.Cu") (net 4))
 (segment (start 51.7525 70.8025) (end 51.7525 67.31) (width 1.905) (layer "B.Cu") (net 4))
 (segment (start 46.6725 64.77) (end 44.1325 64.77) (width 1.905) (layer "B.Cu") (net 4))
 (segment (start 57.785 67.31) (end 56.832501 67.31) (width 1.905) (layer "B.Cu") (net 1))
 (segment (start 61.912499 64.769999) (end 61.9125 64.77) (width 0.2) (layer "B.Cu") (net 1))
 (segment (start 60.325 64.77) (end 57.785 67.31) (width 1.905) (layer "B.Cu") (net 1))
 (segment (start 56.832501 67.31) (end 54.2925 67.31) (width 1.905) (layer "B.Cu") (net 1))
 (segment (start 61.9125 64.77) (end 60.325 64.77) (width 1.905) (layer "B.Cu") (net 1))
 (segment (start 53.0225 64.77) (end 48.26 60.0075) (width 1.905) (layer "B.Cu") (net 2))
 (segment (start 38.1 55.245) (end 39.0525 55.245) (width 1.905) (layer "B.Cu") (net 2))
 (segment (start 36.83 56.515) (end 38.1 55.245) (width 1.905) (layer "B.Cu") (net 2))
 (segment (start 56.832501 64.77) (end 54.2925 64.77) (width 1.905) (layer "B.Cu") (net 2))
 (segment (start 54.2925 64.77) (end 53.0225 64.77) (width 1.905) (layer "B.Cu") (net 2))
 (segment (start 48.26 60.0075) (end 38.1 60.0075) (width 1.905) (layer "B.Cu") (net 2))
 (segment (start 36.83 58.7375) (end 36.83 56.515) (width 1.905) (layer "B.Cu") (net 2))
 (segment (start 36.83 58.7375) (end 38.1 60.0075) (width 1.905) (layer "B.Cu") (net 2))
 (segment (start 46.6725 52.705) (end 42.8625 52.705) (width 1.905) (layer "B.Cu") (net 11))
 (segment (start 42.8625 52.705) (end 40.3225 50.165) (width 1.905) (layer "B.Cu") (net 11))
 (segment (start 40.3225 50.165) (end 39.0525 50.165) (width 1.905) (layer "B.Cu") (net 11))
 (segment (start 42.8625 55.245) (end 46.6725 55.245) (width 1.905) (layer "B.Cu") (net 12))
 (segment (start 39.0525 57.785) (end 40.3225 57.785) (width 1.905) (layer "B.Cu") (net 12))
 (segment (start 40.3225 57.785) (end 42.8625 55.245) (width 1.905) (layer "B.Cu") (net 12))
 (segment (start 62.23 45.72) (end 64.135 47.625) (width 1.905) (layer "B.Cu") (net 10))
 (segment (start 44.1325 50.165) (end 46.6725 50.165) (width 1.905) (layer "B.Cu") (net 10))
 (segment (start 64.135 47.625) (end 64.135 54.2925) (width 1.905) (layer "B.Cu") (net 10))
 (segment (start 64.135 54.2925) (end 68.8975 59.055) (width 1.905) (layer "B.Cu") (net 10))
 (segment (start 68.8975 76.835) (end 64.4525 81.28) (width 1.905) (layer "B.Cu") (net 10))
 (segment (start 46.6725 50.165) (end 51.1175 45.72) (width 1.905) (layer "B.Cu") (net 10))
 (segment (start 68.8975 59.055) (end 68.8975 76.835) (width 1.905) (layer "B.Cu") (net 10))
 (segment (start 51.1175 45.72) (end 62.23 45.72) (width 1.905) (layer "B.Cu") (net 10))
 (segment (start 56.832501 69.85) (end 54.2925 69.85) (width 1.905) (layer "B.Cu") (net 7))
 (segment (start 56.832501 69.85) (end 56.832501 72.350001) (width 1.905) (layer "B.Cu") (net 7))
 (segment (start 56.8325 81.28) (end 56.8325 79.375) (width 1.905) (layer "B.Cu") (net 9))
 (segment (start 56.8325 79.375) (end 61.9125 74.295) (width 1.905) (layer "B.Cu") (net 9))
 (segment (start 61.9125 74.295) (end 61.9125 72.39) (width 1.905) (layer "B.Cu") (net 9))
 (segment (start 56.8325 55.245) (end 61.9125 55.245) (width 0.6) (layer "F.Cu") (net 8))
 (via (at 56.8325 55.245) (size 1.905) (drill 0.6) (layers "F.Cu" "B.Cu") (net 8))
 (via (at 61.9125 55.245) (size 1.905) (drill 0.6) (layers "F.Cu" "B.Cu") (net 8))
 (segment (start 54.2925 50.165) (end 56.8325 50.165) (width 1.905) (layer "B.Cu") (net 8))
 (segment (start 61.9125 80.645) (end 61.9125 81.28) (width 1.905) (layer "B.Cu") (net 8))
 (segment (start 54.2925 62.23) (end 51.7525 59.69) (width 1.905) (layer "B.Cu") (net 8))
 (segment (start 53.0225 50.165) (end 54.2925 50.165) (width 1.905) (layer "B.Cu") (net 8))
 (segment (start 56.8325 50.165) (end 56.8325 55.245) (width 1.905) (layer "B.Cu") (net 8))
 (segment (start 51.7525 51.435) (end 53.0225 50.165) (width 1.905) (layer "B.Cu") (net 8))
 (segment (start 61.9125 55.245) (end 66.675 60.0075) (width 1.905) (layer "B.Cu") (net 8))
 (segment (start 51.7525 59.69) (end 51.7525 51.435) (width 1.905) (layer "B.Cu") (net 8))
 (segment (start 56.8325 62.23) (end 54.2925 62.23) (width 1.905) (layer "B.Cu") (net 8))
 (segment (start 66.675 60.0075) (end 66.675 75.8825) (width 1.905) (layer "B.Cu") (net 8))
 (segment (start 66.675 75.8825) (end 61.9125 80.645) (width 1.905) (layer "B.Cu") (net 8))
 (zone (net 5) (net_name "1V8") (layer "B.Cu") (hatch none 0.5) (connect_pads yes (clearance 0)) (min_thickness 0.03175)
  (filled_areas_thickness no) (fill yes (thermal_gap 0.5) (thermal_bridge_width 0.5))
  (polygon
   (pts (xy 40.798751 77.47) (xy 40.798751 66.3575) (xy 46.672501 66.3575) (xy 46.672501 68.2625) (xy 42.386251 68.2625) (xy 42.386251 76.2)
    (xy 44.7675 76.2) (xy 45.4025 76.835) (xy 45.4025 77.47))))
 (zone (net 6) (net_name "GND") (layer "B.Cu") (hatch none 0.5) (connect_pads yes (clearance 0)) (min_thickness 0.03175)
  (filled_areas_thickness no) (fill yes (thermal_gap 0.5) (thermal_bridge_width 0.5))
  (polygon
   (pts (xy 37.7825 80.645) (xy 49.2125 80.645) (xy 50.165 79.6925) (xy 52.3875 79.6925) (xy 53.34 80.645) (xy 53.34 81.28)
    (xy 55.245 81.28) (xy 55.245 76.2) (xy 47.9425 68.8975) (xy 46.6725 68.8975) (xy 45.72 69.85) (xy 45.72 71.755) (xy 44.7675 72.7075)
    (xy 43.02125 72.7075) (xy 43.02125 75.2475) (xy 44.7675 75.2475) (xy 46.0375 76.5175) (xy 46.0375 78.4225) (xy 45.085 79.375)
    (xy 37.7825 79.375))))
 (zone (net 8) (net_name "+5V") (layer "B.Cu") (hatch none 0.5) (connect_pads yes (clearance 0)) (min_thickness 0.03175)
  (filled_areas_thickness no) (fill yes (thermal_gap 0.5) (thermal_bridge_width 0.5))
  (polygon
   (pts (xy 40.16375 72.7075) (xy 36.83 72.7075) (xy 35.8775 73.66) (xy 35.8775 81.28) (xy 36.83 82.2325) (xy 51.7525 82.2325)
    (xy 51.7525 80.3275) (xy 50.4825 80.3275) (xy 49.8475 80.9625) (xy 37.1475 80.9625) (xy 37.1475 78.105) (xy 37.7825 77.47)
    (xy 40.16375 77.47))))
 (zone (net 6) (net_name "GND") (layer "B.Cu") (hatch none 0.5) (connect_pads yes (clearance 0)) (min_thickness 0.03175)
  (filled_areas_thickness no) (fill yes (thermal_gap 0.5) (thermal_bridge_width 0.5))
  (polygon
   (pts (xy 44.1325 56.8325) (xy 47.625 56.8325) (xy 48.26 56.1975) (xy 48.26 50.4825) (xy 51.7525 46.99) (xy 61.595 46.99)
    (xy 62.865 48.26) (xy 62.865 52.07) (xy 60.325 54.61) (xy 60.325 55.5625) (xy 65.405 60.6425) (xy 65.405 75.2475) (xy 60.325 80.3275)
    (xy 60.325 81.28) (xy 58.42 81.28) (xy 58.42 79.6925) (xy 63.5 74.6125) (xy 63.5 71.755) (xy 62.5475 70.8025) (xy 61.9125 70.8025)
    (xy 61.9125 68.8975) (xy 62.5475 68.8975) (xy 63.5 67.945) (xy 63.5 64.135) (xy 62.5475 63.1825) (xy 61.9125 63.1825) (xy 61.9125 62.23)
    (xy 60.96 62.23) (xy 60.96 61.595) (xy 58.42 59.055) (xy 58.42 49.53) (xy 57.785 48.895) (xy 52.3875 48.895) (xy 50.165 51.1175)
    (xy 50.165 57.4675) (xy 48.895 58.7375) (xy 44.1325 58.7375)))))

